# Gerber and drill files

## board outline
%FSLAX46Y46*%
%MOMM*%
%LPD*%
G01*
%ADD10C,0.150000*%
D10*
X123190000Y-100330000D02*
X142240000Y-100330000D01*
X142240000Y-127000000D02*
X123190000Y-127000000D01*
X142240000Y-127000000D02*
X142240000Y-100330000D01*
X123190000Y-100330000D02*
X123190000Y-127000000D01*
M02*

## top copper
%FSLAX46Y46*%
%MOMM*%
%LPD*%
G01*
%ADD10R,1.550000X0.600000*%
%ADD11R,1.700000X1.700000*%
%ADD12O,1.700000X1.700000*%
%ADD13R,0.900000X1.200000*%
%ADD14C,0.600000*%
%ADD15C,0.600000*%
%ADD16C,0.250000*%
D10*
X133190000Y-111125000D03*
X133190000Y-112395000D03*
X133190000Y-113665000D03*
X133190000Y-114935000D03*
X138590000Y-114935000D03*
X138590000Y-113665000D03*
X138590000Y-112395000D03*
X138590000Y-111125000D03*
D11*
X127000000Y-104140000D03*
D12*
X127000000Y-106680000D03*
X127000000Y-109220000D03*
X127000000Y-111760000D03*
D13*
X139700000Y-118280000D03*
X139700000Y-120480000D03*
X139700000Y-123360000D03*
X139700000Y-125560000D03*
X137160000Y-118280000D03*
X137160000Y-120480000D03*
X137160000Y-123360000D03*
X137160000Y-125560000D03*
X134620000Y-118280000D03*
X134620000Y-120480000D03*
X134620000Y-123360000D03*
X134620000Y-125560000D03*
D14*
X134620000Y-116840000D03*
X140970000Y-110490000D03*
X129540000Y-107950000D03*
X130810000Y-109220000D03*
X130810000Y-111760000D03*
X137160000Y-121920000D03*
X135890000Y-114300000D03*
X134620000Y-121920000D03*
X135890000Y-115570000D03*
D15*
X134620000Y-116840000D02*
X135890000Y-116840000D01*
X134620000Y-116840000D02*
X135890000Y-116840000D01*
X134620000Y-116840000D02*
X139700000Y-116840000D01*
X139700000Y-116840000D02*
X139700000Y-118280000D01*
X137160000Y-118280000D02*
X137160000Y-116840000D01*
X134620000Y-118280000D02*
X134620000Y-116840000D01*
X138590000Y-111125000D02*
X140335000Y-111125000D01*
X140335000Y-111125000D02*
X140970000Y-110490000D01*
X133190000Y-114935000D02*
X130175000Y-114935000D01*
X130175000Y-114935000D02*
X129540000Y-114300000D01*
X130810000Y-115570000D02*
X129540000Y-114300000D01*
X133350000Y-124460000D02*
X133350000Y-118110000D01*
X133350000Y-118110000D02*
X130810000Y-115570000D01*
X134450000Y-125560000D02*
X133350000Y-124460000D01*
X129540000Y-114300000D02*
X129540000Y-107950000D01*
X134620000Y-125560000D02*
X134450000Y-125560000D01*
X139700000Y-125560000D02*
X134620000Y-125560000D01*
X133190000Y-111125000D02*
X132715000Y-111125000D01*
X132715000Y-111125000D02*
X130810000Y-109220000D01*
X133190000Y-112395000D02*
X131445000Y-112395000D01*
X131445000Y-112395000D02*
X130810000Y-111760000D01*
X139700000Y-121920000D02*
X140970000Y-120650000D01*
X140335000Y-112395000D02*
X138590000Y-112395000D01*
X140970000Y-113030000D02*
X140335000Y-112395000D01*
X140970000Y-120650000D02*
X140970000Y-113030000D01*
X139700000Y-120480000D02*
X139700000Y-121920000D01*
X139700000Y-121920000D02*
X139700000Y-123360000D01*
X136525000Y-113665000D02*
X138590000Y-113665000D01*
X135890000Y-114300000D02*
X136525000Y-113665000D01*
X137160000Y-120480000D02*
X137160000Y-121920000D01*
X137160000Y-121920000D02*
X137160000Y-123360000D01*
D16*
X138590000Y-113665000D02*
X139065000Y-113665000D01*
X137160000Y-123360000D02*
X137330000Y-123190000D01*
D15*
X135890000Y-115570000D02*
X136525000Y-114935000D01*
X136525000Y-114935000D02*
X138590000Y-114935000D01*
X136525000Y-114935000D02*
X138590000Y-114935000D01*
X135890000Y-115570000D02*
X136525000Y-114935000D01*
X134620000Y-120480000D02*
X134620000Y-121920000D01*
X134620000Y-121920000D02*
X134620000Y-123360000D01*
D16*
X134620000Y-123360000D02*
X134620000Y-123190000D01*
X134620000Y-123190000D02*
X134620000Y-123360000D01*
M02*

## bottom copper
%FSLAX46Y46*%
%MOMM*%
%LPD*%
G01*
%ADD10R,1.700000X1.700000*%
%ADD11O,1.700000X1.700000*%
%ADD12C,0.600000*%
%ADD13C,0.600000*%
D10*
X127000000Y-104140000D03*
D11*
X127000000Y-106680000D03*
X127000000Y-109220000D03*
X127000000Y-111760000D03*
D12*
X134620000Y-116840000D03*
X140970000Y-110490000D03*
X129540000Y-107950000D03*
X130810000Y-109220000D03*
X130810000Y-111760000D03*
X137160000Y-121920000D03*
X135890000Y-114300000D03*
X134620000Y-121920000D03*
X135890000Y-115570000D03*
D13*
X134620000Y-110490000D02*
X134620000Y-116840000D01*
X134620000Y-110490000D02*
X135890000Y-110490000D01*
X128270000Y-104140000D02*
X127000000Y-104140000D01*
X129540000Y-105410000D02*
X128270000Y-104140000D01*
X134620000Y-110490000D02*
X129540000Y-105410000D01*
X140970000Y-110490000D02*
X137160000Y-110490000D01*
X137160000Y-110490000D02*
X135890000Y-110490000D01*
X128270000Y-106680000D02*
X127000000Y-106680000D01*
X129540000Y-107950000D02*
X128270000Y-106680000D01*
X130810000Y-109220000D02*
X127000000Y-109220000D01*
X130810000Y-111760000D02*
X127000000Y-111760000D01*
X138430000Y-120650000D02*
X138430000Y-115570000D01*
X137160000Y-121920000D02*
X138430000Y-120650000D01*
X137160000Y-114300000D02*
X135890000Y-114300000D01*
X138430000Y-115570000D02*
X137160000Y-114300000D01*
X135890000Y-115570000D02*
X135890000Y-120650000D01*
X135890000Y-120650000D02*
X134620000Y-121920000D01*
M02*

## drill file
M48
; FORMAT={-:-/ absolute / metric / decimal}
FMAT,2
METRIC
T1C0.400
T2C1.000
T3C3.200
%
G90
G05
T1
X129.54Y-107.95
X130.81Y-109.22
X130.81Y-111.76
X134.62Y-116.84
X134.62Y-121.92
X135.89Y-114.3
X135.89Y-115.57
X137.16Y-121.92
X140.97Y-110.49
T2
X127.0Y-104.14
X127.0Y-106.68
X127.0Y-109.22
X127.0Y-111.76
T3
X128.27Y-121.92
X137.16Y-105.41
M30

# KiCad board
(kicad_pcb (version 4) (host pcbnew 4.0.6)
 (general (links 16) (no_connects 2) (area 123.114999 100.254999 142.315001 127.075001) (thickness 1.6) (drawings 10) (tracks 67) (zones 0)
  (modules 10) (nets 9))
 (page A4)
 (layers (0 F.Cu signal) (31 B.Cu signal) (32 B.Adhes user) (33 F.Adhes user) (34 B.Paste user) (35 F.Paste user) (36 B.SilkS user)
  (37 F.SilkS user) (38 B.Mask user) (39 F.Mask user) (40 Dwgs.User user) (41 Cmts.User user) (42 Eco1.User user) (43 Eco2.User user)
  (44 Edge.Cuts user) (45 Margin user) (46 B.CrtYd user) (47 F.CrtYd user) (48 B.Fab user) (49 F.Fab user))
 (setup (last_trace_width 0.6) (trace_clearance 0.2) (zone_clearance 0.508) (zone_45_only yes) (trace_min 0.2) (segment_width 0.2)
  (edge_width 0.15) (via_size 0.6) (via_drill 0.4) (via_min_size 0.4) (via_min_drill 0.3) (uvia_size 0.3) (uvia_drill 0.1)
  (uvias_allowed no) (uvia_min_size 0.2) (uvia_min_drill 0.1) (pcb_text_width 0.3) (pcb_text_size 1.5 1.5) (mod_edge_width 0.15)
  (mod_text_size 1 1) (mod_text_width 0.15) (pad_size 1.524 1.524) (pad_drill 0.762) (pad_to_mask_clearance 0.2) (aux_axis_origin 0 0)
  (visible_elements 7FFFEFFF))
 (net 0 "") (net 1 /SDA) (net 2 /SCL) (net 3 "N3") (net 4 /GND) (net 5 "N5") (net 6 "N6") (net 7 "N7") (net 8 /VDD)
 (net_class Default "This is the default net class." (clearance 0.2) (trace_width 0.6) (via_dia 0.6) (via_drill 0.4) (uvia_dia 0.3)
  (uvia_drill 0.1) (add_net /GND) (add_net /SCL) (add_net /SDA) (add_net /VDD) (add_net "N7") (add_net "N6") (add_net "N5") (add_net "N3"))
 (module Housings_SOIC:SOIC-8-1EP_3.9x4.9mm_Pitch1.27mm (layer F.Cu) (at 135.89 113.03)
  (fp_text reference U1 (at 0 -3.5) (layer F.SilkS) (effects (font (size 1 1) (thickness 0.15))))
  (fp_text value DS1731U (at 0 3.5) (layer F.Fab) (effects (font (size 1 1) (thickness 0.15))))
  (pad 1 smd rect (at -2.7 -1.905) (size 1.55 0.6) (layers F.Cu F.Paste F.Mask) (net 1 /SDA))
  (pad 2 smd rect (at -2.7 -0.635) (size 1.55 0.6) (layers F.Cu F.Paste F.Mask) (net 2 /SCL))
  (pad 3 smd rect (at -2.7 0.635) (size 1.55 0.6) (layers F.Cu F.Paste F.Mask) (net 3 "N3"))
  (pad 4 smd rect (at -2.7 1.905) (size 1.55 0.6) (layers F.Cu F.Paste F.Mask) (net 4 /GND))
  (pad 5 smd rect (at 2.7 1.905) (size 1.55 0.6) (layers F.Cu F.Paste F.Mask) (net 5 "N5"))
  (pad 6 smd rect (at 2.7 0.635) (size 1.55 0.6) (layers F.Cu F.Paste F.Mask) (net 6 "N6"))
  (pad 7 smd rect (at 2.7 -0.635) (size 1.55 0.6) (layers F.Cu F.Paste F.Mask) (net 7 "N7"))
  (pad 8 smd rect (at 2.7 -1.905) (size 1.55 0.6) (layers F.Cu F.Paste F.Mask) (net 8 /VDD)))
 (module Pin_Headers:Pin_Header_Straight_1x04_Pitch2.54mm (layer F.Cu) (at 127 104.14)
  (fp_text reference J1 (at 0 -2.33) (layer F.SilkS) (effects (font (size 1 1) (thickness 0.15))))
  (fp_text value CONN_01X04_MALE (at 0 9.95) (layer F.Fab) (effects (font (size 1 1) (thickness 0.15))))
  (pad 1 thru_hole rect (at 0 0) (size 1.7 1.7) (drill 1) (layers *.Cu *.Mask) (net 8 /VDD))
  (pad 2 thru_hole oval (at 0 2.54) (size 1.7 1.7) (drill 1) (layers *.Cu *.Mask) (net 4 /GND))
  (pad 3 thru_hole oval (at 0 5.08) (size 1.7 1.7) (drill 1) (layers *.Cu *.Mask) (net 1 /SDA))
  (pad 4 thru_hole oval (at 0 7.62) (size 1.7 1.7) (drill 1) (layers *.Cu *.Mask) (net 2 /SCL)))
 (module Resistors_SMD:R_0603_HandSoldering (layer F.Cu) (at 139.7 119.38 270)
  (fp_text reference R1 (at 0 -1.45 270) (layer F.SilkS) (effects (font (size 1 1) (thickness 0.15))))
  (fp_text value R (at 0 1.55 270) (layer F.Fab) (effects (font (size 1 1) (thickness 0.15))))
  (pad 1 smd rect (at -1.1 0 270) (size 1.2 0.9) (layers F.Cu F.Paste F.Mask) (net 8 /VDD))
  (pad 2 smd rect (at 1.1 0 270) (size 1.2 0.9) (layers F.Cu F.Paste F.Mask) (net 7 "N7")))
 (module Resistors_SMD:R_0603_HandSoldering (layer F.Cu) (at 139.7 124.46 270)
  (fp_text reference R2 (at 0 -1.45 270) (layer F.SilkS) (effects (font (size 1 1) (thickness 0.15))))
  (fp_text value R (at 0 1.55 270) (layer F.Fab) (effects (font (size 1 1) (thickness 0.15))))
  (pad 1 smd rect (at -1.1 0 270) (size 1.2 0.9) (layers F.Cu F.Paste F.Mask) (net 7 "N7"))
  (pad 2 smd rect (at 1.1 0 270) (size 1.2 0.9) (layers F.Cu F.Paste F.Mask) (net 4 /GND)))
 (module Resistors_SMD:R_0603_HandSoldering (layer F.Cu) (at 137.16 119.38 270)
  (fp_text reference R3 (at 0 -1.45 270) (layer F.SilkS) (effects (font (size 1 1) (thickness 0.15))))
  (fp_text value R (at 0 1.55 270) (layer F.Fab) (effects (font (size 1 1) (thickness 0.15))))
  (pad 1 smd rect (at -1.1 0 270) (size 1.2 0.9) (layers F.Cu F.Paste F.Mask) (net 8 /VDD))
  (pad 2 smd rect (at 1.1 0 270) (size 1.2 0.9) (layers F.Cu F.Paste F.Mask) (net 6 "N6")))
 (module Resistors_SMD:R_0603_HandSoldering (layer F.Cu) (at 137.16 124.46 270)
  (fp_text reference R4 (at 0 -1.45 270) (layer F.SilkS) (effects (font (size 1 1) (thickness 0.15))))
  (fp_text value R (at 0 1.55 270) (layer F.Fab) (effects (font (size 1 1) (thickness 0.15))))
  (pad 1 smd rect (at -1.1 0 270) (size 1.2 0.9) (layers F.Cu F.Paste F.Mask) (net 6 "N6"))
  (pad 2 smd rect (at 1.1 0 270) (size 1.2 0.9) (layers F.Cu F.Paste F.Mask) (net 4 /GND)))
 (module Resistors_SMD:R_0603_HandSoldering (layer F.Cu) (at 134.62 119.38 270)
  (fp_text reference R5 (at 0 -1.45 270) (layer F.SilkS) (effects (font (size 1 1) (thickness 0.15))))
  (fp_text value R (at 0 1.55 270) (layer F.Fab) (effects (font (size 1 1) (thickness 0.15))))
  (pad 1 smd rect (at -1.1 0 270) (size 1.2 0.9) (layers F.Cu F.Paste F.Mask) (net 8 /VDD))
  (pad 2 smd rect (at 1.1 0 270) (size 1.2 0.9) (layers F.Cu F.Paste F.Mask) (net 5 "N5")))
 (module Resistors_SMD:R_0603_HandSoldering (layer F.Cu) (at 134.62 124.46 270)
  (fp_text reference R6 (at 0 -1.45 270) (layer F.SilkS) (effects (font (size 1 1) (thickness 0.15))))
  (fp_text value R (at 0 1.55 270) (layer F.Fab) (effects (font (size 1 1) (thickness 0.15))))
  (pad 1 smd rect (at -1.1 0 270) (size 1.2 0.9) (layers F.Cu F.Paste F.Mask) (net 5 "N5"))
  (pad 2 smd rect (at 1.1 0 270) (size 1.2 0.9) (layers F.Cu F.Paste F.Mask) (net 4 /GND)))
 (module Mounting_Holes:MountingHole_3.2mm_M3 (layer F.Cu) (at 128.27 121.92)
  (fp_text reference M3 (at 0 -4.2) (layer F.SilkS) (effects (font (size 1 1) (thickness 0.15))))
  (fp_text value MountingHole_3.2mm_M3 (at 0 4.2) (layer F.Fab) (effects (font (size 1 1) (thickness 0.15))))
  (pad 1 np_thru_hole circle (at 0 0) (size 3.2 3.2) (drill 3.2) (layers *.Cu *.Mask)))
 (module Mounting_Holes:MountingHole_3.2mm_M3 (layer F.Cu) (at 137.16 105.41)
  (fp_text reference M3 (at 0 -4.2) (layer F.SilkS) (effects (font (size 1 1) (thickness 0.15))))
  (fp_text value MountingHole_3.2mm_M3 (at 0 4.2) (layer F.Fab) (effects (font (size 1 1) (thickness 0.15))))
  (pad 1 np_thru_hole circle (at 0 0) (size 3.2 3.2) (drill 3.2) (layers *.Cu *.Mask)))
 (gr_line (start 123.19 100.33) (end 142.24 100.33) (angle 90) (layer Edge.Cuts) (width 0.15))
 (gr_line (start 142.24 127) (end 123.19 127) (angle 90) (layer Edge.Cuts) (width 0.15))
 (gr_line (start 142.24 127) (end 142.24 100.33) (angle 90) (layer Edge.Cuts) (width 0.15))
 (gr_line (start 123.19 100.33) (end 123.19 127) (angle 90) (layer Edge.Cuts) (width 0.15))
 (segment (start 134.62 110.49) (end 134.62 116.84) (width 0.6) (layer B.Cu) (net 8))
 (via (at 134.62 116.84) (size 0.6) (drill 0.4) (layers F.Cu B.Cu) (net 8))
 (segment (start 134.62 116.84) (end 135.89 116.84) (width 0.6) (layer F.Cu) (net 8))
 (segment (start 134.62 116.84) (end 135.89 116.84) (width 0.6) (layer F.Cu) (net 8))
 (segment (start 134.62 116.84) (end 139.7 116.84) (width 0.6) (layer F.Cu) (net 8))
 (segment (start 139.7 116.84) (end 139.7 118.28) (width 0.6) (layer F.Cu) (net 8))
 (segment (start 137.16 118.28) (end 137.16 116.84) (width 0.6) (layer F.Cu) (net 8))
 (segment (start 134.62 118.28) (end 134.62 116.84) (width 0.6) (layer F.Cu) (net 8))
 (segment (start 134.62 110.49) (end 135.89 110.49) (width 0.6) (layer B.Cu) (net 8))
 (segment (start 138.59 111.125) (end 140.335 111.125) (width 0.6) (layer F.Cu) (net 8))
 (segment (start 128.27 104.14) (end 127 104.14) (width 0.6) (layer B.Cu) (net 8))
 (segment (start 129.54 105.41) (end 128.27 104.14) (width 0.6) (layer B.Cu) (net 8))
 (segment (start 134.62 110.49) (end 129.54 105.41) (width 0.6) (layer B.Cu) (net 8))
 (segment (start 140.97 110.49) (end 137.16 110.49) (width 0.6) (layer B.Cu) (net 8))
 (segment (start 137.16 110.49) (end 135.89 110.49) (width 0.6) (layer B.Cu) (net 8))
 (via (at 140.97 110.49) (size 0.6) (drill 0.4) (layers F.Cu B.Cu) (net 8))
 (segment (start 140.335 111.125) (end 140.97 110.49) (width 0.6) (layer F.Cu) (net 8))
 (segment (start 133.19 114.935) (end 130.175 114.935) (width 0.6) (layer F.Cu) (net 4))
 (segment (start 130.175 114.935) (end 129.54 114.3) (width 0.6) (layer F.Cu) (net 4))
 (segment (start 130.81 115.57) (end 129.54 114.3) (width 0.6) (layer F.Cu) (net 4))
 (segment (start 133.35 124.46) (end 133.35 118.11) (width 0.6) (layer F.Cu) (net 4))
 (segment (start 133.35 118.11) (end 130.81 115.57) (width 0.6) (layer F.Cu) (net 4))
 (segment (start 134.45 125.56) (end 133.35 124.46) (width 0.6) (layer F.Cu) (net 4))
 (segment (start 128.27 106.68) (end 127 106.68) (width 0.6) (layer B.Cu) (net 4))
 (segment (start 129.54 107.95) (end 128.27 106.68) (width 0.6) (layer B.Cu) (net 4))
 (via (at 129.54 107.95) (size 0.6) (drill 0.4) (layers F.Cu B.Cu) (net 4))
 (segment (start 129.54 114.3) (end 129.54 107.95) (width 0.6) (layer F.Cu) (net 4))
 (segment (start 134.62 125.56) (end 134.45 125.56) (width 0.6) (layer F.Cu) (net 4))
 (segment (start 139.7 125.56) (end 134.62 125.56) (width 0.6) (layer F.Cu) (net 4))
 (segment (start 133.19 111.125) (end 132.715 111.125) (width 0.6) (layer F.Cu) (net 1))
 (segment (start 132.715 111.125) (end 130.81 109.22) (width 0.6) (layer F.Cu) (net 1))
 (segment (start 130.81 109.22) (end 127 109.22) (width 0.6) (layer B.Cu) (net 1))
 (via (at 130.81 109.22) (size 0.6) (drill 0.4) (layers F.Cu B.Cu) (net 1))
 (segment (start 133.19 112.395) (end 131.445 112.395) (width 0.6) (layer F.Cu) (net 2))
 (segment (start 130.81 111.76) (end 127 111.76) (width 0.6) (layer B.Cu) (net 2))
 (via (at 130.81 111.76) (size 0.6) (drill 0.4) (layers F.Cu B.Cu) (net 2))
 (segment (start 131.445 112.395) (end 130.81 111.76) (width 0.6) (layer F.Cu) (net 2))
 (segment (start 139.7 121.92) (end 140.97 120.65) (width 0.6) (layer F.Cu) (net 7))
 (segment (start 140.335 112.395) (end 138.59 112.395) (width 0.6) (layer F.Cu) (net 7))
 (segment (start 140.97 113.03) (end 140.335 112.395) (width 0.6) (layer F.Cu) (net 7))
 (segment (start 140.97 120.65) (end 140.97 113.03) (width 0.6) (layer F.Cu) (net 7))
 (segment (start 139.7 120.48) (end 139.7 121.92) (width 0.6) (layer F.Cu) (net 7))
 (segment (start 139.7 121.92) (end 139.7 123.36) (width 0.6) (layer F.Cu) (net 7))
 (segment (start 138.43 120.65) (end 138.43 115.57) (width 0.6) (layer B.Cu) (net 6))
 (segment (start 137.16 121.92) (end 138.43 120.65) (width 0.6) (layer B.Cu) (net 6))
 (via (at 137.16 121.92) (size 0.6) (drill 0.4) (layers F.Cu B.Cu) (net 6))
 (segment (start 136.525 113.665) (end 138.59 113.665) (width 0.6) (layer F.Cu) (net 6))
 (segment (start 135.89 114.3) (end 136.525 113.665) (width 0.6) (layer F.Cu) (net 6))
 (via (at 135.89 114.3) (size 0.6) (drill 0.4) (layers F.Cu B.Cu) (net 6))
 (segment (start 137.16 114.3) (end 135.89 114.3) (width 0.6) (layer B.Cu) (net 6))
 (segment (start 138.43 115.57) (end 137.16 114.3) (width 0.6) (layer B.Cu) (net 6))
 (segment (start 137.16 120.48) (end 137.16 121.92) (width 0.6) (layer F.Cu) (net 6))
 (segment (start 137.16 121.92) (end 137.16 123.36) (width 0.6) (layer F.Cu) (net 6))
 (segment (start 138.59 113.665) (end 139.065 113.665) (width 0.25) (layer F.Cu) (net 6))
 (segment (start 137.16 123.36) (end 137.33 123.19) (width 0.25) (layer F.Cu) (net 6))
 (via (at 134.62 121.92) (size 0.6) (drill 0.4) (layers F.Cu B.Cu) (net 5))
 (via (at 135.89 115.57) (size 0.6) (drill 0.4) (layers F.Cu B.Cu) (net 5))
 (segment (start 135.89 115.57) (end 135.89 120.65) (width 0.6) (layer B.Cu) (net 5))
 (segment (start 135.89 120.65) (end 134.62 121.92) (width 0.6) (layer B.Cu) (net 5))
 (segment (start 135.89 115.57) (end 136.525 114.935) (width 0.6) (layer F.Cu) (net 5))
 (segment (start 136.525 114.935) (end 138.59 114.935) (width 0.6) (layer F.Cu) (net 5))
 (segment (start 136.525 114.935) (end 138.59 114.935) (width 0.6) (layer F.Cu) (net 5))
 (segment (start 135.89 115.57) (end 136.525 114.935) (width 0.6) (layer F.Cu) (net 5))
 (segment (start 134.62 120.48) (end 134.62 121.92) (width 0.6) (layer F.Cu) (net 5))
 (segment (start 134.62 121.92) (end 134.62 123.36) (width 0.6) (layer F.Cu) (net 5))
 (segment (start 134.62 123.36) (end 134.62 123.19) (width 0.25) (layer F.Cu) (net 5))
 (segment (start 134.62 123.19) (end 134.62 123.36) (width 0.25) (layer F.Cu) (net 5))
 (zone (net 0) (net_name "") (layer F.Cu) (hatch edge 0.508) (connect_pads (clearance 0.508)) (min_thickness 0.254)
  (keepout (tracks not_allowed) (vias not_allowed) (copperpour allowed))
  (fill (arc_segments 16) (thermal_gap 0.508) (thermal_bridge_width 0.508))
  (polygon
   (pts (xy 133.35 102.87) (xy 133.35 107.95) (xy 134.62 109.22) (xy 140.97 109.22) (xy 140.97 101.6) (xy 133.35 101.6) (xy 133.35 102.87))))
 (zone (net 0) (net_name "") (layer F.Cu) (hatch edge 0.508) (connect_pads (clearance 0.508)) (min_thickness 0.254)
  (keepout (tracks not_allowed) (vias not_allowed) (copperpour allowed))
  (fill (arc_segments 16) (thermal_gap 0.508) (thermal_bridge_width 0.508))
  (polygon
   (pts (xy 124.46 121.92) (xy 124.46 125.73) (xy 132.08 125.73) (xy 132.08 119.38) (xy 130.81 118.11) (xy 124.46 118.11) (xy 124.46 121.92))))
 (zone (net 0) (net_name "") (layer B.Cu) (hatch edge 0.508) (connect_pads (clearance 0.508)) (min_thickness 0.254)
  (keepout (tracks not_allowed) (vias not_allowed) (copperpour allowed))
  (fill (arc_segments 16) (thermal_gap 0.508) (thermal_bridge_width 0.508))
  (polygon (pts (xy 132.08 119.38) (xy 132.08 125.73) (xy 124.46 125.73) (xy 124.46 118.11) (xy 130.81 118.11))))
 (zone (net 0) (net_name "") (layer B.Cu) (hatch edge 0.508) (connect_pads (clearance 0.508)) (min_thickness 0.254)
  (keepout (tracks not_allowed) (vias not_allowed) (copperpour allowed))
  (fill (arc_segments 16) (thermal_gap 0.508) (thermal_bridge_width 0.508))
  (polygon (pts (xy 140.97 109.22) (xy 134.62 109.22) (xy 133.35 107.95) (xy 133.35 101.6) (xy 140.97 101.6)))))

